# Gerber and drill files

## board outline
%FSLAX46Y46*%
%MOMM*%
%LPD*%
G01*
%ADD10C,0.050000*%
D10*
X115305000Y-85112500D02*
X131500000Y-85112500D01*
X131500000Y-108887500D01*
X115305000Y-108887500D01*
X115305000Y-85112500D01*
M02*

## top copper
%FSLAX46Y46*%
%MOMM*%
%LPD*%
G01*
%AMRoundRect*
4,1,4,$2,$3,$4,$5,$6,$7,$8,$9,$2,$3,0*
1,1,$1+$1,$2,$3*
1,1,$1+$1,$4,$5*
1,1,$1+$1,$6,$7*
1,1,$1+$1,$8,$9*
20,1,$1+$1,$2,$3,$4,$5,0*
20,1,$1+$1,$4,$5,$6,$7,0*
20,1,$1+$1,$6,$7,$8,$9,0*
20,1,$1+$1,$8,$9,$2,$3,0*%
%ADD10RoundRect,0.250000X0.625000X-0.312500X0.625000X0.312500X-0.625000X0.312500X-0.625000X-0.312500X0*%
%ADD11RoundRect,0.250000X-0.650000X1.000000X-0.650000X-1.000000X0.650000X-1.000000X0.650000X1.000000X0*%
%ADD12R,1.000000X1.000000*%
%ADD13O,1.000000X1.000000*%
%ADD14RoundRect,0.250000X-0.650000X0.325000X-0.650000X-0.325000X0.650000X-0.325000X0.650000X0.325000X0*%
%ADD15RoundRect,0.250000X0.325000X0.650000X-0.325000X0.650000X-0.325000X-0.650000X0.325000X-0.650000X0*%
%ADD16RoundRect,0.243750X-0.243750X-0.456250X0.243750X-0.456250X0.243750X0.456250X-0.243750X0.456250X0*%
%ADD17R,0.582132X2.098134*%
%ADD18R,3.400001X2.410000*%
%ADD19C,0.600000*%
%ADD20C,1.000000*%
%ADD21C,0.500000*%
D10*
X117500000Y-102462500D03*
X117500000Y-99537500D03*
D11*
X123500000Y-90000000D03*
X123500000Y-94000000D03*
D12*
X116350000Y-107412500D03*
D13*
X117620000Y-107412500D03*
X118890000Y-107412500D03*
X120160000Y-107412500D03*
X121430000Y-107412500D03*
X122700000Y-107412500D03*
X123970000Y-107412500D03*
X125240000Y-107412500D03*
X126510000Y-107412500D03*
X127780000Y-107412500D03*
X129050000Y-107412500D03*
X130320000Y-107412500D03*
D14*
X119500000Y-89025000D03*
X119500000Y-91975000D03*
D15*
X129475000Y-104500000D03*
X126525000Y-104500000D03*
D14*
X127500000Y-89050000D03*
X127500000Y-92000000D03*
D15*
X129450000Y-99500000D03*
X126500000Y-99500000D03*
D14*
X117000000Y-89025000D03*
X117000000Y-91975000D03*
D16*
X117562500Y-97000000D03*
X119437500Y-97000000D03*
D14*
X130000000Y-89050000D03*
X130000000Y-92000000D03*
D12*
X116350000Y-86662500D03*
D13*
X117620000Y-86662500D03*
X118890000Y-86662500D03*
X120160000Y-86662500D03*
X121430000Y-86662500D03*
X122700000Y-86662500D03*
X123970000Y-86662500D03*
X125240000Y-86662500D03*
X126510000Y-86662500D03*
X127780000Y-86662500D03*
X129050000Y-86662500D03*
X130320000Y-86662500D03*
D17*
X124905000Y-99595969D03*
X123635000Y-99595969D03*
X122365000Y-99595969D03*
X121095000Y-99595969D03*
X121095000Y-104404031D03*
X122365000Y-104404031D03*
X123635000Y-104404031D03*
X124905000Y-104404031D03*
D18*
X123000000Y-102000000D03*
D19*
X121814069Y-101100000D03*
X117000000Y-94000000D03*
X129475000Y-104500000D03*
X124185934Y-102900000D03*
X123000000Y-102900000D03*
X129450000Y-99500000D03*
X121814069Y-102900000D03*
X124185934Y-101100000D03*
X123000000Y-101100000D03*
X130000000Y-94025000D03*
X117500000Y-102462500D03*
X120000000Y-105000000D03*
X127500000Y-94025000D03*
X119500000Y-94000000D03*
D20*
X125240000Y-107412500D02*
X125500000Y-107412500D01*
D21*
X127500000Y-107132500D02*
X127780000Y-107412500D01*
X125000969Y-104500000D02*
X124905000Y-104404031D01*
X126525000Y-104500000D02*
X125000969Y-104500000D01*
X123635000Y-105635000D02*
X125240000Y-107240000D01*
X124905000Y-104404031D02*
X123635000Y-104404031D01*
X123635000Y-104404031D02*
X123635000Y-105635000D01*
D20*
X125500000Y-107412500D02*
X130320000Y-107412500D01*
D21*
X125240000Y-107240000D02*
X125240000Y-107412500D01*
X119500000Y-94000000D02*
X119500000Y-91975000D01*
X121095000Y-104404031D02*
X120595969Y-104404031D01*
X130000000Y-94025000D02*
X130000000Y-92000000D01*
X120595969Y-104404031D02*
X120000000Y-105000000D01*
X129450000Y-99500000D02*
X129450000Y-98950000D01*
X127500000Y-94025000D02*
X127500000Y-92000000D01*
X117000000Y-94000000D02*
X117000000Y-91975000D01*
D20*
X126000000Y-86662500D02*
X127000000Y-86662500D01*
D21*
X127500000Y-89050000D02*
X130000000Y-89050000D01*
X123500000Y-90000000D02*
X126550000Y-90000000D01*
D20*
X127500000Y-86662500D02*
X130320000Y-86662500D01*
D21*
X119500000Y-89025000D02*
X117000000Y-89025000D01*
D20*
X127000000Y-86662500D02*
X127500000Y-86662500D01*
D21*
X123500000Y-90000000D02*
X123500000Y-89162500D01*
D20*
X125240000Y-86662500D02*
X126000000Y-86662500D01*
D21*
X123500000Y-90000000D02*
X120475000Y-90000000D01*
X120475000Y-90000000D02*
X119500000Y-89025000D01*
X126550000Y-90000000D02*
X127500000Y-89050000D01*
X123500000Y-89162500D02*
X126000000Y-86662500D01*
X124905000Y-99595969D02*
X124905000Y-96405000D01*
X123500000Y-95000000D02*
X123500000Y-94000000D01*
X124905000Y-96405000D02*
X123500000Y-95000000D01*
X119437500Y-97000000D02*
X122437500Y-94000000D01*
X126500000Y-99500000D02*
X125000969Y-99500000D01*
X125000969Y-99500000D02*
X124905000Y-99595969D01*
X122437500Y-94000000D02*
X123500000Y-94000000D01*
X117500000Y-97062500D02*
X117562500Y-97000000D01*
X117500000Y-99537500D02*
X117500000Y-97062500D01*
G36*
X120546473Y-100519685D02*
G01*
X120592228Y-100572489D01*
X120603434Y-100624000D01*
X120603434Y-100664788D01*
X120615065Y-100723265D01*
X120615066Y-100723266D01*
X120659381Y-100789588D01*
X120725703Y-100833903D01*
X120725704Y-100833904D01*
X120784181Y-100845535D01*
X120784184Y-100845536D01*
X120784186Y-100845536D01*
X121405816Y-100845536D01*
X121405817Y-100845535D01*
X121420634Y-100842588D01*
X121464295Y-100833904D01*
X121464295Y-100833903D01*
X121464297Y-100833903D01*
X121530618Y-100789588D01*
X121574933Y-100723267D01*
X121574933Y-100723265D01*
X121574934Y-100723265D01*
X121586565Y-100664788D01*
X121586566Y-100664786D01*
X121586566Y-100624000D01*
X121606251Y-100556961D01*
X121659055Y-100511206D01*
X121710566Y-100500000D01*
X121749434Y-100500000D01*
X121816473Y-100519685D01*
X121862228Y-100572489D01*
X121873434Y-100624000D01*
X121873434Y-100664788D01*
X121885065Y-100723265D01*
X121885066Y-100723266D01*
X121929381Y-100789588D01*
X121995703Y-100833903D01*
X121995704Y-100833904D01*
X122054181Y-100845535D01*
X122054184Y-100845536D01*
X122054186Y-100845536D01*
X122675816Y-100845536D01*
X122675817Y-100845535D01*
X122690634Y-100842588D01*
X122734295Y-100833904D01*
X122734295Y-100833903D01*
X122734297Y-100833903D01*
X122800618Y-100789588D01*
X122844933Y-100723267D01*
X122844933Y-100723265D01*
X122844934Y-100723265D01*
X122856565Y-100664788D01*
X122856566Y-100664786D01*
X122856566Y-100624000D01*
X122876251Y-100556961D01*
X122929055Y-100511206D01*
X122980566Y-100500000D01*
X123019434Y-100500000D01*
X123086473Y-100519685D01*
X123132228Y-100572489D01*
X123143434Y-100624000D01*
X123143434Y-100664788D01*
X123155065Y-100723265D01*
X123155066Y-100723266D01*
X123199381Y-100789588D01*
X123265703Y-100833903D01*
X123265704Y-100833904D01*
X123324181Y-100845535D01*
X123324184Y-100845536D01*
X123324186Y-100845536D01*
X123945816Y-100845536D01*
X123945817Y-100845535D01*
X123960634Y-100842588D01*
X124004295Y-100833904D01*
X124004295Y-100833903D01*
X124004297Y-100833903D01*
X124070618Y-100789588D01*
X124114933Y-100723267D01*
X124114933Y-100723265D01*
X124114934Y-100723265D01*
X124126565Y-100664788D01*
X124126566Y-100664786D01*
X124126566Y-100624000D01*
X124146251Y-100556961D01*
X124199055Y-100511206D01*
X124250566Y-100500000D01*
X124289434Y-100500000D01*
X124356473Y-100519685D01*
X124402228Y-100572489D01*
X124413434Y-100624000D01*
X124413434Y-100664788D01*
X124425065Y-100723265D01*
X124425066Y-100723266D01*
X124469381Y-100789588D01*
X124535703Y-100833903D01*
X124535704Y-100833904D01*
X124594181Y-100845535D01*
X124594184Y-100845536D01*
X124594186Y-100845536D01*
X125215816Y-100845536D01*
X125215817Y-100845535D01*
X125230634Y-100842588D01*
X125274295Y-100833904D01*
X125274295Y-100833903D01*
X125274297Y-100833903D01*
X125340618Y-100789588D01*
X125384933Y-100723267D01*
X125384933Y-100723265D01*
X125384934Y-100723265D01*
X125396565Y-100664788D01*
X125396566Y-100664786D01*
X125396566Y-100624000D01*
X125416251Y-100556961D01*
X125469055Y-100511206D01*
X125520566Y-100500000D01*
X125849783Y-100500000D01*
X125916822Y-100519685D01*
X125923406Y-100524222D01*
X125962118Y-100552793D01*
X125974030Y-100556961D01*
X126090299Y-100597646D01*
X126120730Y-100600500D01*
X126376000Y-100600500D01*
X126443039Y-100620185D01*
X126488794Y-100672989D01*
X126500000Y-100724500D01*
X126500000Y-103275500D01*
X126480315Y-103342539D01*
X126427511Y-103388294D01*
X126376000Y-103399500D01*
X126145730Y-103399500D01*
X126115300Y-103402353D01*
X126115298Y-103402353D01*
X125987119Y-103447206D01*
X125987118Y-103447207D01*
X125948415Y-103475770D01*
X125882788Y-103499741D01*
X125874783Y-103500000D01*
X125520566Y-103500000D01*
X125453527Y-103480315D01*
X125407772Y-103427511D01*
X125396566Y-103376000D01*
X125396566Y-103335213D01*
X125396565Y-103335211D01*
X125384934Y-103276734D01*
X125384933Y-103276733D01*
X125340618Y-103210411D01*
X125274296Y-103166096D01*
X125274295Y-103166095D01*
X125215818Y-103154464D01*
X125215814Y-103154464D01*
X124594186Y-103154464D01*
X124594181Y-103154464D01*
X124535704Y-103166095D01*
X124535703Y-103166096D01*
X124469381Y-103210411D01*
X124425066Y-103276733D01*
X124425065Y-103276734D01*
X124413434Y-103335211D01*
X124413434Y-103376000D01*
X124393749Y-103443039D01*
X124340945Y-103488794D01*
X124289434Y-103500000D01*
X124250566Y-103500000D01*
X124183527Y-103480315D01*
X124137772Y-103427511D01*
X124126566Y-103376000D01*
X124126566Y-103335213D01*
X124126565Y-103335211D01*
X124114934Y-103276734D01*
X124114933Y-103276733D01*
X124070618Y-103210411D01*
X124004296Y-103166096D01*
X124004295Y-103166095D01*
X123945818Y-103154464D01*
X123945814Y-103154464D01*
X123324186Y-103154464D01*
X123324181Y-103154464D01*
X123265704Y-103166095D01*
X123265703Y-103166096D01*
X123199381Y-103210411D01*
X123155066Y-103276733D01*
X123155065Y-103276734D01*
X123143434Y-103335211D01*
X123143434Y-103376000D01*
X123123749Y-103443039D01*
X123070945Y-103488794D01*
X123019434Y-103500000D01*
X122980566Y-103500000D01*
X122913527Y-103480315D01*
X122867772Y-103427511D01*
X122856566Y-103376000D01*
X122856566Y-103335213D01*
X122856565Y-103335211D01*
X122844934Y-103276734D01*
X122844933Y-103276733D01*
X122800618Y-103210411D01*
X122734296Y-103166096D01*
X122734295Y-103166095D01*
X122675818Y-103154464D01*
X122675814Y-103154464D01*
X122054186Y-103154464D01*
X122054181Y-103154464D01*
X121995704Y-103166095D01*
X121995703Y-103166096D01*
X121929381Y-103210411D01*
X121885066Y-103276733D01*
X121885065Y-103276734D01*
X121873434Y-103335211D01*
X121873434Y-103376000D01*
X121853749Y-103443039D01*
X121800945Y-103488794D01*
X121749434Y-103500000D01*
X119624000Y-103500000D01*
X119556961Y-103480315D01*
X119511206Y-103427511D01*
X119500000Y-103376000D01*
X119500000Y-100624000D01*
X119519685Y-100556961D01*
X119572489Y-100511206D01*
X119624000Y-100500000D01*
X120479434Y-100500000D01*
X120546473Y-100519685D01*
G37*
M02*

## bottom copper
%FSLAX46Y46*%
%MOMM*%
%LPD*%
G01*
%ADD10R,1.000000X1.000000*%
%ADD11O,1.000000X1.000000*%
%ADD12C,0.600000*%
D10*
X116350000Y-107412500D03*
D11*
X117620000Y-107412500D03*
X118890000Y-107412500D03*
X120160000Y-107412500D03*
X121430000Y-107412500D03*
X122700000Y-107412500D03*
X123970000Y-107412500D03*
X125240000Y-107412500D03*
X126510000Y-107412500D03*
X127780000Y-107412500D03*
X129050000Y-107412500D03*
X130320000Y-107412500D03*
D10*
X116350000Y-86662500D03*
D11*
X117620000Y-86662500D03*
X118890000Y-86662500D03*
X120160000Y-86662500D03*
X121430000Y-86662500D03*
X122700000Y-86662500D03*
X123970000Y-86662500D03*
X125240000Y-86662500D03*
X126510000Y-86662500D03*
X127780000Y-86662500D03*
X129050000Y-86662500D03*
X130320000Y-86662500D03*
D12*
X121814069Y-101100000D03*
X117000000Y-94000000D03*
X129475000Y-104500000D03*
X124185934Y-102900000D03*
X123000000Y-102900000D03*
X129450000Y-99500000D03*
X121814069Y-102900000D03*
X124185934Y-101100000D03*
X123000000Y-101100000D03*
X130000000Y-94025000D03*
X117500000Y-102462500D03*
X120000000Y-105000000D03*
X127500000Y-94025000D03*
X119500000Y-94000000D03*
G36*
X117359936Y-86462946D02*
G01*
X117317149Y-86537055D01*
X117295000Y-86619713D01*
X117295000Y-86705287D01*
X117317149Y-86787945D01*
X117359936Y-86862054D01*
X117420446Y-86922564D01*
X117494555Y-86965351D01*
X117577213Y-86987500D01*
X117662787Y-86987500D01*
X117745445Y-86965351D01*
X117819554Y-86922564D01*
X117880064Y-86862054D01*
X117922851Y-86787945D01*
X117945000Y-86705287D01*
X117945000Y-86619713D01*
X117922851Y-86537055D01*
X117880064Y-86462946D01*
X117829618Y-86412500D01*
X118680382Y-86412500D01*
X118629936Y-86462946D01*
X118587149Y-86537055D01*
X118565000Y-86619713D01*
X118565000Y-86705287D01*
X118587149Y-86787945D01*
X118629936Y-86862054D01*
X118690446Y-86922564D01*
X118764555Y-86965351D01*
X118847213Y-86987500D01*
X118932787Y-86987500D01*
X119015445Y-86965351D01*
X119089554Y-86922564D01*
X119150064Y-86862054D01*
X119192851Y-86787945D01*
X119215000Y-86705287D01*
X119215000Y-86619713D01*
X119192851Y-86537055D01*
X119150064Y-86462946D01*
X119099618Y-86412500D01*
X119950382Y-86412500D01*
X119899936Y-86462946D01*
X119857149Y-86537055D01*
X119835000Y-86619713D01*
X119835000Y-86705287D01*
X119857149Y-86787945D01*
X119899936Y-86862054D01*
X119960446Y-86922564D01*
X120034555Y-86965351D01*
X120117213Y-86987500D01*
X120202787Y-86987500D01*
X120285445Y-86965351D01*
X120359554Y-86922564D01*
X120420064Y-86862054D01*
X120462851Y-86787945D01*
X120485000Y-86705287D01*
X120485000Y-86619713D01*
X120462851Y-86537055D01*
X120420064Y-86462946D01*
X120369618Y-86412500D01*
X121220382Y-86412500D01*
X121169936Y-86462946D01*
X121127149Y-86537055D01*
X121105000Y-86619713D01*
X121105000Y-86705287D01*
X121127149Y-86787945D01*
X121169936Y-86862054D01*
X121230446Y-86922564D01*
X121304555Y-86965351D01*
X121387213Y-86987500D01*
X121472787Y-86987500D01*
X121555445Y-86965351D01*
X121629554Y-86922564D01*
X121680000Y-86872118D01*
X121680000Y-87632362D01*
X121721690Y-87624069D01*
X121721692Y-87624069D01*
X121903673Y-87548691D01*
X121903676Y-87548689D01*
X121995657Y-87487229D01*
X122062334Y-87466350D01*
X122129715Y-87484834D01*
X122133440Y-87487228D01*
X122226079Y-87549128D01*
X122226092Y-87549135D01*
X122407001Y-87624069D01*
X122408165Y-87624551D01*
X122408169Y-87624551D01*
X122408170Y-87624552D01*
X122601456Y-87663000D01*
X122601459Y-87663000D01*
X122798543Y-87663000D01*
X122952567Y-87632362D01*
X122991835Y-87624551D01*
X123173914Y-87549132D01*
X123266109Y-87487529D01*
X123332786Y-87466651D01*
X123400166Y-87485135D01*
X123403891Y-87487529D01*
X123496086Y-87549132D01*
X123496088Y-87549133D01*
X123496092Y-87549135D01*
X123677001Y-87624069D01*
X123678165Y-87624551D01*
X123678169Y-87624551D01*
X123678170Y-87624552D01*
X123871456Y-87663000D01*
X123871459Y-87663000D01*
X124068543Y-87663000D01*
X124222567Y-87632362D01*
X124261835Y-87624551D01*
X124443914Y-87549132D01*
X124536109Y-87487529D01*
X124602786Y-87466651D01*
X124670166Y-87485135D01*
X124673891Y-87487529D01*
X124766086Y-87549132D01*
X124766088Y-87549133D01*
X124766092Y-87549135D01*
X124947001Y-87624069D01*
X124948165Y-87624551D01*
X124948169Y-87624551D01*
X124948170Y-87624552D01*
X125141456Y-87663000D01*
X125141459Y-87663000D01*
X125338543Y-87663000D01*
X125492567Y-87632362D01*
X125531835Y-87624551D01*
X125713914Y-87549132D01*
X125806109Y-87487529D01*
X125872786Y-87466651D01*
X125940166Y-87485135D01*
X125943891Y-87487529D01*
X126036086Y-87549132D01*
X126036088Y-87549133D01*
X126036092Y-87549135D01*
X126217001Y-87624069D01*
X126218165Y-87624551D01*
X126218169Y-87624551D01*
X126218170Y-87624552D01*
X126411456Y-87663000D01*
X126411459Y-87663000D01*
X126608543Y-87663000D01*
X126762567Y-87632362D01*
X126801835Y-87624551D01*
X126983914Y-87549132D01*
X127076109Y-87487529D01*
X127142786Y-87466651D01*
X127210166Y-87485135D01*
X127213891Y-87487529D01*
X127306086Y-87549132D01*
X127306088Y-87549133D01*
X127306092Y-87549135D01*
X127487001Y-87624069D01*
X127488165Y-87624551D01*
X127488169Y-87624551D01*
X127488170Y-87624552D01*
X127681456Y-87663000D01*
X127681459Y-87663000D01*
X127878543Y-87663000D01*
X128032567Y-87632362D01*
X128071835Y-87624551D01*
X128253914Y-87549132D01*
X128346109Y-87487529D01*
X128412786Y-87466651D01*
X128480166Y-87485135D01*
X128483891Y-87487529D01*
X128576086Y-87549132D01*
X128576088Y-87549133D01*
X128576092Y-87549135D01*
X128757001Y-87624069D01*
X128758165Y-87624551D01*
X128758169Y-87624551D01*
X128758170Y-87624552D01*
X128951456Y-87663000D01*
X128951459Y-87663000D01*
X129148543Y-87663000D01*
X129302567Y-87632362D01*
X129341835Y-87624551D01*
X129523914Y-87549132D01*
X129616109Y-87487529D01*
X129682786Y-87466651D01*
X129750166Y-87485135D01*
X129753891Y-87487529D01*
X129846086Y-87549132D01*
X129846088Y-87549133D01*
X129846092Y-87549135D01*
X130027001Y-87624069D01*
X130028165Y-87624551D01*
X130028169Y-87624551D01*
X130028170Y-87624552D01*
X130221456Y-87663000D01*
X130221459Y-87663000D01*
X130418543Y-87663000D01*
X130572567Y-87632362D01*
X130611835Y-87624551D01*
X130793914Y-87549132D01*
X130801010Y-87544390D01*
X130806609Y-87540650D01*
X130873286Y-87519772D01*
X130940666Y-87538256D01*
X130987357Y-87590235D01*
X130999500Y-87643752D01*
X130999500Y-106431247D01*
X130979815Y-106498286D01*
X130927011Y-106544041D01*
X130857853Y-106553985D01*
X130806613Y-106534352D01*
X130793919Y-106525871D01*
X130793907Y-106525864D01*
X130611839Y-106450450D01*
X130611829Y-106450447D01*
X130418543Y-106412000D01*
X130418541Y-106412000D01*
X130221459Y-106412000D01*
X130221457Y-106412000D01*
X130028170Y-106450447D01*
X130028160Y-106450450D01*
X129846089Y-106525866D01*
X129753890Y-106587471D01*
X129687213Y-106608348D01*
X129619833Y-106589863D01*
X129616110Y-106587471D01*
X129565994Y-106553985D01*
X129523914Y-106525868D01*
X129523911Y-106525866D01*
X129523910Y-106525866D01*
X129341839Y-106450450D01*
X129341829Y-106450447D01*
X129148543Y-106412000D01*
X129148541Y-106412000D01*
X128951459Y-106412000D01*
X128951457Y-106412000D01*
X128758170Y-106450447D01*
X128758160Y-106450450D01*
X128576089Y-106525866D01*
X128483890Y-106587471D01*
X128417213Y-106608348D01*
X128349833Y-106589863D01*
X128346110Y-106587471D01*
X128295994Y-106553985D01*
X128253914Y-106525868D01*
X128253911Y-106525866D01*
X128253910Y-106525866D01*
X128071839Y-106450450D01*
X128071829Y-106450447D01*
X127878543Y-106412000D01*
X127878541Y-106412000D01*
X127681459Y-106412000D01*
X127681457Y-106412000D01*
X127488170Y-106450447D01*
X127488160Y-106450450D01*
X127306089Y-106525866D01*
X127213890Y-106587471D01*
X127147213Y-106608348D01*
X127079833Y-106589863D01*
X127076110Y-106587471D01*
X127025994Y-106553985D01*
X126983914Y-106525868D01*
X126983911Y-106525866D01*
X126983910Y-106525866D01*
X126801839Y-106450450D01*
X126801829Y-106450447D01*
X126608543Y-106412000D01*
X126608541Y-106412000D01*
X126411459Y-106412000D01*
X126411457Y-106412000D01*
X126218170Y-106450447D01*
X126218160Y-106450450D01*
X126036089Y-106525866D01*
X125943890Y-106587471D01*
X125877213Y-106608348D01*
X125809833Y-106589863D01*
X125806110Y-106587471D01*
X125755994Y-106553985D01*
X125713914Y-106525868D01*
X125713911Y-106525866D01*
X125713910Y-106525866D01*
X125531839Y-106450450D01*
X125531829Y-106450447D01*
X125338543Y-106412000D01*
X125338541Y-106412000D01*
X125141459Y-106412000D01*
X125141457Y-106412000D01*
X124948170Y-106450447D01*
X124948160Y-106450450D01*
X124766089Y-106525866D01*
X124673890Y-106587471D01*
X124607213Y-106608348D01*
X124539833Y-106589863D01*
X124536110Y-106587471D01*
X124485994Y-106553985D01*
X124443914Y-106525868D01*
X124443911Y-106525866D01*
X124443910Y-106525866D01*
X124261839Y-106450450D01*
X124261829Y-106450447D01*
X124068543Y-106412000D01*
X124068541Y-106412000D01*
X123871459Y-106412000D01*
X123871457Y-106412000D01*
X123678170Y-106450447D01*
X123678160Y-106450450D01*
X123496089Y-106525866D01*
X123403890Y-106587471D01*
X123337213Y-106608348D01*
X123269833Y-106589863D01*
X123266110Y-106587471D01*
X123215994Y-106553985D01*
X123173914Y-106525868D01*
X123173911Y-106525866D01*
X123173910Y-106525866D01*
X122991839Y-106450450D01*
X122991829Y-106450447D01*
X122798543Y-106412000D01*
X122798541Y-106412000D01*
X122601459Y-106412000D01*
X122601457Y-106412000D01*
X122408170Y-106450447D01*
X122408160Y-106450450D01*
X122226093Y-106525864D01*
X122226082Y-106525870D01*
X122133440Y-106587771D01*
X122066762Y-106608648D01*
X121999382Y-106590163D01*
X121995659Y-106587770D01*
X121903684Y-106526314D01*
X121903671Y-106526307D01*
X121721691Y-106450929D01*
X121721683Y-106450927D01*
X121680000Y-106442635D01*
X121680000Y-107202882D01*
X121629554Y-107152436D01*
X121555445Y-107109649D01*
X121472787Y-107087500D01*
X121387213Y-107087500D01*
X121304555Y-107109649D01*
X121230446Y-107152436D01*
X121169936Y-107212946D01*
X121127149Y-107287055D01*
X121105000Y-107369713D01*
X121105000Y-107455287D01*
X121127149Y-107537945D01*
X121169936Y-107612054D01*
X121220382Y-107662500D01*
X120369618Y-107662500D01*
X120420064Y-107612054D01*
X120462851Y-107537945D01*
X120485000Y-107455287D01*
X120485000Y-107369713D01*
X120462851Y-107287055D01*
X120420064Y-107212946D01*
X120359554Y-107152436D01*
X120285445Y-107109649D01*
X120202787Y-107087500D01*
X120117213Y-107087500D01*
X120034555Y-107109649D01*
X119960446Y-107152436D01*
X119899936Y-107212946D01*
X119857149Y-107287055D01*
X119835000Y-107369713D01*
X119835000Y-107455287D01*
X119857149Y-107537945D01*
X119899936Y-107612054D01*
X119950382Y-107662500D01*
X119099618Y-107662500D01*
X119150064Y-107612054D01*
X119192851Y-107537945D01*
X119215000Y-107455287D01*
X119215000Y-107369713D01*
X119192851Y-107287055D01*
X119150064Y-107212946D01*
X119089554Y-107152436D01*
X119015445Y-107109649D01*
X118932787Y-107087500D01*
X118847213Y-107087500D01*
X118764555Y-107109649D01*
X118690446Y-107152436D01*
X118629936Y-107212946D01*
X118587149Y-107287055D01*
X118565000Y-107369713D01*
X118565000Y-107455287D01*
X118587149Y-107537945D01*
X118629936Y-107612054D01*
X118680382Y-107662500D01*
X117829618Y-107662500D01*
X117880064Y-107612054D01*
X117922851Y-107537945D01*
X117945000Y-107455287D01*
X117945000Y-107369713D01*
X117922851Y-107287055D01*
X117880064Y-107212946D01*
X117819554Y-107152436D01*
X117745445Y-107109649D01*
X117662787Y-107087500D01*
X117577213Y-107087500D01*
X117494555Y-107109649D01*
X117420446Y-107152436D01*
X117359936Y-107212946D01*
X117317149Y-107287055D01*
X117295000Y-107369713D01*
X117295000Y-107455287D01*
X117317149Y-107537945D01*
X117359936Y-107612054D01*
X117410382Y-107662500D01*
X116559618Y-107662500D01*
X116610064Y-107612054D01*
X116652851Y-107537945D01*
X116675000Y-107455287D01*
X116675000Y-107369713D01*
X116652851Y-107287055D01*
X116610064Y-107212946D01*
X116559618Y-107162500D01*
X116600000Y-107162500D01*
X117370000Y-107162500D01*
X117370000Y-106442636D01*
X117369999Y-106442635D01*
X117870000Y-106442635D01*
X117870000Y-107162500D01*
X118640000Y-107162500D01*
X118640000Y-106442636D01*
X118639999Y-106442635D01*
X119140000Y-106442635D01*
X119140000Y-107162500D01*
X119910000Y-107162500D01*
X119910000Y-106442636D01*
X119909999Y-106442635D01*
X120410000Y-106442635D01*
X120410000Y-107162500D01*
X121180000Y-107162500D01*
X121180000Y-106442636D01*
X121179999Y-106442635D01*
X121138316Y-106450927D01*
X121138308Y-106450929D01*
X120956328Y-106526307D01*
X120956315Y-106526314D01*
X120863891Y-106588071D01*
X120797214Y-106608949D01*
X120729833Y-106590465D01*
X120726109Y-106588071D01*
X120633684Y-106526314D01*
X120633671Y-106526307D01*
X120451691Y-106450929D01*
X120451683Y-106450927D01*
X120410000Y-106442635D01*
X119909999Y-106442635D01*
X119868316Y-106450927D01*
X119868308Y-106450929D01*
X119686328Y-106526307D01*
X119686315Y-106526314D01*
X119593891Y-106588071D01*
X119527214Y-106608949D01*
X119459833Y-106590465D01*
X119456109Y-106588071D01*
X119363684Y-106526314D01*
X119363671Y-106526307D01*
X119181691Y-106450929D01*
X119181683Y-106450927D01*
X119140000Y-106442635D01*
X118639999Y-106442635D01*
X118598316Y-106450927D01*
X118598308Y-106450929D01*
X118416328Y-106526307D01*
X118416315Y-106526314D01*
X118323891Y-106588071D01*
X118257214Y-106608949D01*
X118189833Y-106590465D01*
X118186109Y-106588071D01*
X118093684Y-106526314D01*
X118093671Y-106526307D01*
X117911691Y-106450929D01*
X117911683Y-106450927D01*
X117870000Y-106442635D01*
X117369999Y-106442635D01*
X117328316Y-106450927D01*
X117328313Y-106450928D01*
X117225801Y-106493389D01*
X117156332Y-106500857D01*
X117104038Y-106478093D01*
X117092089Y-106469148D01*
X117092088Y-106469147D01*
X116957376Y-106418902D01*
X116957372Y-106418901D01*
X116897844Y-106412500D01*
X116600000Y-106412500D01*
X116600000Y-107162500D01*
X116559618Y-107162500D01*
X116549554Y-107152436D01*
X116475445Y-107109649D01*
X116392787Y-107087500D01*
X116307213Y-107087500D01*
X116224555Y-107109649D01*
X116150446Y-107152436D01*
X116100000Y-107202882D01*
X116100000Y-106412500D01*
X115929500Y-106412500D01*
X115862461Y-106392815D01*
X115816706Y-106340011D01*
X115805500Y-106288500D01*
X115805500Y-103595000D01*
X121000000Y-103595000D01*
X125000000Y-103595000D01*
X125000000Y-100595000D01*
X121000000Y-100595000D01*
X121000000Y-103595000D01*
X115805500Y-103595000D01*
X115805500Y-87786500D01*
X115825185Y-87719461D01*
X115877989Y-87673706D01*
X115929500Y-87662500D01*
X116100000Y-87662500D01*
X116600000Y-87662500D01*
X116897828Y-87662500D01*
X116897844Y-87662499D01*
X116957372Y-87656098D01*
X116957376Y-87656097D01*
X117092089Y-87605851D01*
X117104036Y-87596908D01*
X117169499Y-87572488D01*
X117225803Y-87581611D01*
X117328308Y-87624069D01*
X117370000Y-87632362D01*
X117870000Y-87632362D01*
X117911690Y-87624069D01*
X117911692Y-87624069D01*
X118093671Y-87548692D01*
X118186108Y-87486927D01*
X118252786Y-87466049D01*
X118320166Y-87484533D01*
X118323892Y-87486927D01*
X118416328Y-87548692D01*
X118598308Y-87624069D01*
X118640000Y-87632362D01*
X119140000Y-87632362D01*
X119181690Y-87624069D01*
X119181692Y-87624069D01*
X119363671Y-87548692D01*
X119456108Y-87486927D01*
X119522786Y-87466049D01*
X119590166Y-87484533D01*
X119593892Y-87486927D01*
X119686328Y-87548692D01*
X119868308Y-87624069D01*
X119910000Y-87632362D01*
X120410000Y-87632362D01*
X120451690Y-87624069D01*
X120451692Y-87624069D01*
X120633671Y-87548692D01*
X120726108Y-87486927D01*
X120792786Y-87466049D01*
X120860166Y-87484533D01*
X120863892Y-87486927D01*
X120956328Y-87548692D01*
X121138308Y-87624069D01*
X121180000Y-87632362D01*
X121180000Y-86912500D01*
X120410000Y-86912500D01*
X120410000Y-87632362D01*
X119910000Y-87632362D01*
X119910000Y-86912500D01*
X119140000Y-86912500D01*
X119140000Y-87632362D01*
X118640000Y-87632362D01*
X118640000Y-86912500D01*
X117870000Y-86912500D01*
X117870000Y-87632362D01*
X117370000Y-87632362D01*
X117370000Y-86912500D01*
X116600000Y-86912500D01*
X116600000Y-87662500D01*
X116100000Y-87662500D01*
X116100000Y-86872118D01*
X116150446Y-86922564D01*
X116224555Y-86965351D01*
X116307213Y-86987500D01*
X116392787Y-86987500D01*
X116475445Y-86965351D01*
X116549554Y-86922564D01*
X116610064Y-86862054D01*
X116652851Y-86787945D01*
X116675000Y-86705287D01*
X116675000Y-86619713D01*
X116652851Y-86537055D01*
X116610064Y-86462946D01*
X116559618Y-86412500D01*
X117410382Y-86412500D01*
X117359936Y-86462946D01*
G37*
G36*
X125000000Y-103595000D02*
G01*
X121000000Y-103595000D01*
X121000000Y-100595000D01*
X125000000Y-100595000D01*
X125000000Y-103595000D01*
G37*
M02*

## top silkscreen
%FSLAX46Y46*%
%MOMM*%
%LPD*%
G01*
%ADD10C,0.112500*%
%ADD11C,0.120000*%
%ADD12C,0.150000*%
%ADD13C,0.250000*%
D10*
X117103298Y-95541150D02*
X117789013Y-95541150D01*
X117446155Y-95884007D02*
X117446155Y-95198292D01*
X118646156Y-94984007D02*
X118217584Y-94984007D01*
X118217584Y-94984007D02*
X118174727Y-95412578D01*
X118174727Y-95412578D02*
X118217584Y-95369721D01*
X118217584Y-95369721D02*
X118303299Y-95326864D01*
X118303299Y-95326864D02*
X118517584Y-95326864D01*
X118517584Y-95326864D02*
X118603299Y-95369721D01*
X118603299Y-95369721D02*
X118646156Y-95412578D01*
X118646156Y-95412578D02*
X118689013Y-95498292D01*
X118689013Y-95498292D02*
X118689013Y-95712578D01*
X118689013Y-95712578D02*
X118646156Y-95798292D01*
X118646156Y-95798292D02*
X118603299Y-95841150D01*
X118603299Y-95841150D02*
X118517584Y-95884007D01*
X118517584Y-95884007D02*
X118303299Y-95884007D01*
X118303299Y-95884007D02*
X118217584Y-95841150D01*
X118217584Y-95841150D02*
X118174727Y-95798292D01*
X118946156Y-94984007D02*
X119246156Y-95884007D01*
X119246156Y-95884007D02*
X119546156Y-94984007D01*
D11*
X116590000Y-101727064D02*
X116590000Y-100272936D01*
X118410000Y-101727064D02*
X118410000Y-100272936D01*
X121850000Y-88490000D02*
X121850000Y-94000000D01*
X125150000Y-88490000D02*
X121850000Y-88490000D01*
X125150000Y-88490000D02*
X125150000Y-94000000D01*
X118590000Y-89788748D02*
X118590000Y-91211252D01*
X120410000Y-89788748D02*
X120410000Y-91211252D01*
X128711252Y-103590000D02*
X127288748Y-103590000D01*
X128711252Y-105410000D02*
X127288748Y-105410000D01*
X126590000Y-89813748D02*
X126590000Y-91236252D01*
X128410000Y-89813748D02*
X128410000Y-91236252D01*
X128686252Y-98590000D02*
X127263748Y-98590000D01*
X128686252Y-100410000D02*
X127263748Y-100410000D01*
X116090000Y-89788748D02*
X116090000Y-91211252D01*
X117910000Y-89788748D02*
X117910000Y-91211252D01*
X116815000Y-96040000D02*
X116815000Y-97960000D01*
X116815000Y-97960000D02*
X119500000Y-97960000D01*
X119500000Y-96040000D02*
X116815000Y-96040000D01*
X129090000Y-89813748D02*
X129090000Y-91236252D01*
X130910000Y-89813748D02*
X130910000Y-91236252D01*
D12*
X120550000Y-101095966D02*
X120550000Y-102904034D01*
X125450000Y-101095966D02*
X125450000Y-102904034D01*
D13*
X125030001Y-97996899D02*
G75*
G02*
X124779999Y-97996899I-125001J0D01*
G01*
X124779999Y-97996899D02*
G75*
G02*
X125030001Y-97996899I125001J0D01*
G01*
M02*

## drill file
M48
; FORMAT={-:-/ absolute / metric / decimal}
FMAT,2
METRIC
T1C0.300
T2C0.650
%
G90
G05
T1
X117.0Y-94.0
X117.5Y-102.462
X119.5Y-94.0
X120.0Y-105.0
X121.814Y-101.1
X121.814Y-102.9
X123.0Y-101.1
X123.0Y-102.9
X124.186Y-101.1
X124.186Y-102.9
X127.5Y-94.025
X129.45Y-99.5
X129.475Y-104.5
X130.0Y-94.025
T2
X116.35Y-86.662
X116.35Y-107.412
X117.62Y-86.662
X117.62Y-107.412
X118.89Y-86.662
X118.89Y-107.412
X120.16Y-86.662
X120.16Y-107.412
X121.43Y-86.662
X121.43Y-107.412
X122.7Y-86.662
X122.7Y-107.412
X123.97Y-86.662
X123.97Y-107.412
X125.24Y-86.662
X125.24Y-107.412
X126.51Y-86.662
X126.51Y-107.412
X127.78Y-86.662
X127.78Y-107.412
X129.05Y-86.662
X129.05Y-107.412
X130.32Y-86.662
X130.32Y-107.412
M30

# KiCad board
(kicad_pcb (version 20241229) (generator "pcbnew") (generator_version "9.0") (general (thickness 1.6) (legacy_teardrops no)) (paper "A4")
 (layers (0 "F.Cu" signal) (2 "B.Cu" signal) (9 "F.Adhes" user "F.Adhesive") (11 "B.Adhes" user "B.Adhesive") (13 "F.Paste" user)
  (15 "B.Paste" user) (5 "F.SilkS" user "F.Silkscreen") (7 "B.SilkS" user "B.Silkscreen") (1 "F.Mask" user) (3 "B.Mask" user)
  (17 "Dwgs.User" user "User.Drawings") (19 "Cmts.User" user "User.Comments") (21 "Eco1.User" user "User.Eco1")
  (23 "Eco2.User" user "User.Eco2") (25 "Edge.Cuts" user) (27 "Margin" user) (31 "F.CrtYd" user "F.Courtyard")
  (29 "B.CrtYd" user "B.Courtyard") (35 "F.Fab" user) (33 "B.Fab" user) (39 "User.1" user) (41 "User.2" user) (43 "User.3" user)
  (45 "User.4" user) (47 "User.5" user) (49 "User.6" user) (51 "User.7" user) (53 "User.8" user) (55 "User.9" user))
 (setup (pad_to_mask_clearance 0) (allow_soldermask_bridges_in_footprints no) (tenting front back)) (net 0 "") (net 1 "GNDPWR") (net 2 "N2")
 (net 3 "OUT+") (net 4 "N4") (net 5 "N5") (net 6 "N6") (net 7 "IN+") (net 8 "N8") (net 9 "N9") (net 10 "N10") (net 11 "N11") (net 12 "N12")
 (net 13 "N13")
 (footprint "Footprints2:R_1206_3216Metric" (layer "F.Cu") (at 117.5 101 90)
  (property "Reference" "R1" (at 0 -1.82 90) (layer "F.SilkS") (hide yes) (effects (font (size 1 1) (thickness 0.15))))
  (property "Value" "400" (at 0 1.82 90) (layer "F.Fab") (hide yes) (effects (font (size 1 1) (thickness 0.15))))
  (fp_line (start -0.727064 -0.91) (end 0.727064 -0.91) (stroke (width 0.12) (type solid)) (layer "F.SilkS"))
  (fp_line (start -0.727064 0.91) (end 0.727064 0.91) (stroke (width 0.12) (type solid)) (layer "F.SilkS"))
  (pad "1" smd roundrect (at -1.4625 0 90) (size 1.125 1.75) (layers "F.Cu" "F.Mask" "F.Paste") (roundrect_rratio 0.222222) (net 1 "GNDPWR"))
  (pad "2" smd roundrect (at 1.4625 0 90) (size 1.125 1.75) (layers "F.Cu" "F.Mask" "F.Paste") (roundrect_rratio 0.222222) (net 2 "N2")))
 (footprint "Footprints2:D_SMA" (layer "F.Cu") (at 123.5 92 -90)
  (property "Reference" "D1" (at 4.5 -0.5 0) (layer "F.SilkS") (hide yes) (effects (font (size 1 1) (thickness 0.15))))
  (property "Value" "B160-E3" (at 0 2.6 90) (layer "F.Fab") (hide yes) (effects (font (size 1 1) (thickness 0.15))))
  (fp_line (start -3.51 1.65) (end 2 1.65) (stroke (width 0.12) (type solid)) (layer "F.SilkS"))
  (fp_line (start -3.51 -1.65) (end -3.51 1.65) (stroke (width 0.12) (type solid)) (layer "F.SilkS"))
  (fp_line (start -3.51 -1.65) (end 2 -1.65) (stroke (width 0.12) (type solid)) (layer "F.SilkS"))
  (pad "1" smd roundrect (at -2 0 270) (size 2.5 1.8) (layers "F.Cu" "F.Mask" "F.Paste") (roundrect_rratio 0.1388888889) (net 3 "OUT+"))
  (pad "2" smd roundrect (at 2 0 270) (size 2.5 1.8) (layers "F.Cu" "F.Mask" "F.Paste") (roundrect_rratio 0.1388888889) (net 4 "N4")))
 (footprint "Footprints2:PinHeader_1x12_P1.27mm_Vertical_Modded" (layer "F.Cu") (at 115.28 108.9125 90)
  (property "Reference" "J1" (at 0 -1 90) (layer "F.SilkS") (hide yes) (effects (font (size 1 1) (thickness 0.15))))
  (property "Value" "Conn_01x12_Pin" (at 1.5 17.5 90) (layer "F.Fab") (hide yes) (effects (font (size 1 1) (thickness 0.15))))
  (pad "1" thru_hole rect (at 1.5 1.07 90) (size 1 1) (drill 0.65) (layers "*.Cu" "*.Mask") (remove_unused_layers no) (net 1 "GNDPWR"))
  (pad "2" thru_hole oval (at 1.5 2.34 90) (size 1 1) (drill 0.65) (layers "*.Cu" "*.Mask") (remove_unused_layers no) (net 1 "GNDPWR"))
  (pad "3" thru_hole oval (at 1.5 3.61 90) (size 1 1) (drill 0.65) (layers "*.Cu" "*.Mask") (remove_unused_layers no) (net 1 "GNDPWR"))
  (pad "4" thru_hole oval (at 1.5 4.88 90) (size 1 1) (drill 0.65) (layers "*.Cu" "*.Mask") (remove_unused_layers no) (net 1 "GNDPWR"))
  (pad "5" thru_hole oval (at 1.5 6.15 90) (size 1 1) (drill 0.65) (layers "*.Cu" "*.Mask") (remove_unused_layers no) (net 1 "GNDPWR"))
  (pad "6" thru_hole oval (at 1.5 7.42 90) (size 1 1) (drill 0.65) (layers "*.Cu" "*.Mask") (remove_unused_layers no) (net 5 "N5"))
  (pad "7" thru_hole oval (at 1.5 8.69 90) (size 1 1) (drill 0.65) (layers "*.Cu" "*.Mask") (remove_unused_layers no) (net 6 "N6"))
  (pad "8" thru_hole oval (at 1.5 9.96 90) (size 1 1) (drill 0.65) (layers "*.Cu" "*.Mask") (remove_unused_layers no) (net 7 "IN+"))
  (pad "9" thru_hole oval (at 1.5 11.23 90) (size 1 1) (drill 0.65) (layers "*.Cu" "*.Mask") (remove_unused_layers no) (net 7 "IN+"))
  (pad "10" thru_hole oval (at 1.5 12.5 90) (size 1 1) (drill 0.65) (layers "*.Cu" "*.Mask") (remove_unused_layers no) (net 7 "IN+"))
  (pad "11" thru_hole oval (at 1.5 13.77 90) (size 1 1) (drill 0.65) (layers "*.Cu" "*.Mask") (remove_unused_layers no) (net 7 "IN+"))
  (pad "12" thru_hole oval (at 1.5 15.04 90) (size 1 1) (drill 0.65) (layers "*.Cu" "*.Mask") (remove_unused_layers no) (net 7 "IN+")))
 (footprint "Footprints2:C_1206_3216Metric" (layer "F.Cu") (at 119.5 90.5 -90)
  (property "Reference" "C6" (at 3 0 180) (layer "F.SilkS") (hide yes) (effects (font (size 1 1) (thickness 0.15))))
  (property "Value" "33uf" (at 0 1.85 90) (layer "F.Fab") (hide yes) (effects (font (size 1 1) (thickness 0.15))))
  (fp_line (start -0.711252 0.91) (end 0.711252 0.91) (stroke (width 0.12) (type solid)) (layer "F.SilkS"))
  (fp_line (start -0.711252 -0.91) (end 0.711252 -0.91) (stroke (width 0.12) (type solid)) (layer "F.SilkS"))
  (pad "1" smd roundrect (at -1.475 0 270) (size 1.15 1.8) (layers "F.Cu" "F.Mask" "F.Paste") (roundrect_rratio 0.217391) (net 3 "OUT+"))
  (pad "2" smd roundrect (at 1.475 0 270) (size 1.15 1.8) (layers "F.Cu" "F.Mask" "F.Paste") (roundrect_rratio 0.217391) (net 1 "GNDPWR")))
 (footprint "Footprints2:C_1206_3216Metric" (layer "F.Cu") (at 128 104.5 180)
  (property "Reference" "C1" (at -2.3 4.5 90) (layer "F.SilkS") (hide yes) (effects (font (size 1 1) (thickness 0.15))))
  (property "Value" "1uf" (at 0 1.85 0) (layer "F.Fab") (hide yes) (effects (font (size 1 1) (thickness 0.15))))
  (fp_line (start -0.711252 0.91) (end 0.711252 0.91) (stroke (width 0.12) (type solid)) (layer "F.SilkS"))
  (fp_line (start -0.711252 -0.91) (end 0.711252 -0.91) (stroke (width 0.12) (type solid)) (layer "F.SilkS"))
  (pad "1" smd roundrect (at -1.475 0 180) (size 1.15 1.8) (layers "F.Cu" "F.Mask" "F.Paste") (roundrect_rratio 0.217391) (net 1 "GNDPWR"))
  (pad "2" smd roundrect (at 1.475 0 180) (size 1.15 1.8) (layers "F.Cu" "F.Mask" "F.Paste") (roundrect_rratio 0.217391) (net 7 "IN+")))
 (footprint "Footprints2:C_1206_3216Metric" (layer "F.Cu") (at 127.5 90.525 -90)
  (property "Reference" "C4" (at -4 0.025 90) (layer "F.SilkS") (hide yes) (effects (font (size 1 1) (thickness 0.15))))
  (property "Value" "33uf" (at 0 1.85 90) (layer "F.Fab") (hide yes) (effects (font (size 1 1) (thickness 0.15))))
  (fp_line (start -0.711252 0.91) (end 0.711252 0.91) (stroke (width 0.12) (type solid)) (layer "F.SilkS"))
  (fp_line (start -0.711252 -0.91) (end 0.711252 -0.91) (stroke (width 0.12) (type solid)) (layer "F.SilkS"))
  (pad "1" smd roundrect (at -1.475 0 270) (size 1.15 1.8) (layers "F.Cu" "F.Mask" "F.Paste") (roundrect_rratio 0.217391) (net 3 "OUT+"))
  (pad "2" smd roundrect (at 1.475 0 270) (size 1.15 1.8) (layers "F.Cu" "F.Mask" "F.Paste") (roundrect_rratio 0.217391) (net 1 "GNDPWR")))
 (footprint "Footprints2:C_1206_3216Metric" (layer "F.Cu") (at 127.975 99.5 180)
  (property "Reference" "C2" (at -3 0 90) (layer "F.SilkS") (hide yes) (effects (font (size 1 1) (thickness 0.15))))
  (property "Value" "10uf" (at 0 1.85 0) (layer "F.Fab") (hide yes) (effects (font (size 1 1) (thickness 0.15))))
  (fp_line (start -0.711252 0.91) (end 0.711252 0.91) (stroke (width 0.12) (type solid)) (layer "F.SilkS"))
  (fp_line (start -0.711252 -0.91) (end 0.711252 -0.91) (stroke (width 0.12) (type solid)) (layer "F.SilkS"))
  (pad "1" smd roundrect (at -1.475 0 180) (size 1.15 1.8) (layers "F.Cu" "F.Mask" "F.Paste") (roundrect_rratio 0.217391) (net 1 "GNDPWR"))
  (pad "2" smd roundrect (at 1.475 0 180) (size 1.15 1.8) (layers "F.Cu" "F.Mask" "F.Paste") (roundrect_rratio 0.217391) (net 4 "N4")))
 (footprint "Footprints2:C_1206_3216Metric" (layer "F.Cu") (at 117 90.5 -90)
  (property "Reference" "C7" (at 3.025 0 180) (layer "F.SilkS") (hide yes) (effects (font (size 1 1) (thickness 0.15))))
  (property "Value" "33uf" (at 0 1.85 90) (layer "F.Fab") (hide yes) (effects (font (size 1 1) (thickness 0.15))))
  (fp_line (start -0.711252 0.91) (end 0.711252 0.91) (stroke (width 0.12) (type solid)) (layer "F.SilkS"))
  (fp_line (start -0.711252 -0.91) (end 0.711252 -0.91) (stroke (width 0.12) (type solid)) (layer "F.SilkS"))
  (pad "1" smd roundrect (at -1.475 0 270) (size 1.15 1.8) (layers "F.Cu" "F.Mask" "F.Paste") (roundrect_rratio 0.217391) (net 3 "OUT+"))
  (pad "2" smd roundrect (at 1.475 0 270) (size 1.15 1.8) (layers "F.Cu" "F.Mask" "F.Paste") (roundrect_rratio 0.217391) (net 1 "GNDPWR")))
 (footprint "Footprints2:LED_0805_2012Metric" (layer "F.Cu") (at 118.5 97)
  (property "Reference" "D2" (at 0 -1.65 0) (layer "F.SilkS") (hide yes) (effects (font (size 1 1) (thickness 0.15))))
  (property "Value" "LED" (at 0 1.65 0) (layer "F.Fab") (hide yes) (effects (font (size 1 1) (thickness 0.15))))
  (fp_line (start -1.685 -0.96) (end -1.685 0.96) (stroke (width 0.12) (type solid)) (layer "F.SilkS"))
  (fp_line (start -1.685 0.96) (end 1 0.96) (stroke (width 0.12) (type solid)) (layer "F.SilkS"))
  (fp_line (start 1 -0.96) (end -1.685 -0.96) (stroke (width 0.12) (type solid)) (layer "F.SilkS"))
  (pad "1" smd roundrect (at -0.9375 0) (size 0.975 1.4) (layers "F.Cu" "F.Mask" "F.Paste") (roundrect_rratio 0.25) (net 2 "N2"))
  (pad "2" smd roundrect (at 0.9375 0) (size 0.975 1.4) (layers "F.Cu" "F.Mask" "F.Paste") (roundrect_rratio 0.25) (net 4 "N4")))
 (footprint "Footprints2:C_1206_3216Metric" (layer "F.Cu") (at 130 90.525 -90)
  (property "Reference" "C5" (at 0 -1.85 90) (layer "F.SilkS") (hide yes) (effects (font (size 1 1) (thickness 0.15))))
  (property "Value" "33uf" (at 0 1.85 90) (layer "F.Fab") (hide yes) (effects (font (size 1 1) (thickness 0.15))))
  (fp_line (start -0.711252 0.91) (end 0.711252 0.91) (stroke (width 0.12) (type solid)) (layer "F.SilkS"))
  (fp_line (start -0.711252 -0.91) (end 0.711252 -0.91) (stroke (width 0.12) (type solid)) (layer "F.SilkS"))
  (pad "1" smd roundrect (at -1.475 0 270) (size 1.15 1.8) (layers "F.Cu" "F.Mask" "F.Paste") (roundrect_rratio 0.217391) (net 3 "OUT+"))
  (pad "2" smd roundrect (at 1.475 0 270) (size 1.15 1.8) (layers "F.Cu" "F.Mask" "F.Paste") (roundrect_rratio 0.217391) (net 1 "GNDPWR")))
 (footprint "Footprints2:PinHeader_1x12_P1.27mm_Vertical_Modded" (layer "F.Cu") (at 115.28 88.1625 90)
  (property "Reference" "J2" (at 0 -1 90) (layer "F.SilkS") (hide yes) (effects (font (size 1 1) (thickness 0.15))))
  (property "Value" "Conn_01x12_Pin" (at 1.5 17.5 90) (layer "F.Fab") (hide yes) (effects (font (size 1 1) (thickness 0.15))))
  (pad "1" thru_hole rect (at 1.5 1.07 90) (size 1 1) (drill 0.65) (layers "*.Cu" "*.Mask") (remove_unused_layers no) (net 1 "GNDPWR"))
  (pad "2" thru_hole oval (at 1.5 2.34 90) (size 1 1) (drill 0.65) (layers "*.Cu" "*.Mask") (remove_unused_layers no) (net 1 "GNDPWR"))
  (pad "3" thru_hole oval (at 1.5 3.61 90) (size 1 1) (drill 0.65) (layers "*.Cu" "*.Mask") (remove_unused_layers no) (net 1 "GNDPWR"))
  (pad "4" thru_hole oval (at 1.5 4.88 90) (size 1 1) (drill 0.65) (layers "*.Cu" "*.Mask") (remove_unused_layers no) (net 1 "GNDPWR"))
  (pad "5" thru_hole oval (at 1.5 6.15 90) (size 1 1) (drill 0.65) (layers "*.Cu" "*.Mask") (remove_unused_layers no) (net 1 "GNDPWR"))
  (pad "6" thru_hole oval (at 1.5 7.42 90) (size 1 1) (drill 0.65) (layers "*.Cu" "*.Mask") (remove_unused_layers no) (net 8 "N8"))
  (pad "7" thru_hole oval (at 1.5 8.69 90) (size 1 1) (drill 0.65) (layers "*.Cu" "*.Mask") (remove_unused_layers no) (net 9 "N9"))
  (pad "8" thru_hole oval (at 1.5 9.96 90) (size 1 1) (drill 0.65) (layers "*.Cu" "*.Mask") (remove_unused_layers no) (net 3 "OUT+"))
  (pad "9" thru_hole oval (at 1.5 11.23 90) (size 1 1) (drill 0.65) (layers "*.Cu" "*.Mask") (remove_unused_layers no) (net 3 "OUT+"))
  (pad "10" thru_hole oval (at 1.5 12.5 90) (size 1 1) (drill 0.65) (layers "*.Cu" "*.Mask") (remove_unused_layers no) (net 3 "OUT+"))
  (pad "11" thru_hole oval (at 1.5 13.77 90) (size 1 1) (drill 0.65) (layers "*.Cu" "*.Mask") (remove_unused_layers no) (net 3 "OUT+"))
  (pad "12" thru_hole oval (at 1.5 15.04 90) (size 1 1) (drill 0.65) (layers "*.Cu" "*.Mask") (remove_unused_layers no) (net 3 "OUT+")))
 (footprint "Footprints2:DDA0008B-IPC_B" (layer "F.Cu") (at 123 102 -90)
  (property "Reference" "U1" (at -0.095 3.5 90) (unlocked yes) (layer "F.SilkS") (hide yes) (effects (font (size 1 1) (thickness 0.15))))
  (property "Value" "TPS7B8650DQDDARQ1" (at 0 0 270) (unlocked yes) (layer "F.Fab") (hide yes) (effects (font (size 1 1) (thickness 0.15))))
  (fp_line (start -0.904034 2.45) (end 0.904034 2.45) (stroke (width 0.15) (type solid)) (layer "F.SilkS"))
  (fp_line (start -0.904034 -2.45) (end 0.904034 -2.45) (stroke (width 0.15) (type solid)) (layer "F.SilkS"))
  (fp_circle (center -4.003101 -1.905) (end -3.8781 -1.905) (stroke (width 0.25) (type solid)) (fill no) (layer "F.SilkS"))
  (pad "1" smd rect (at -2.404031 -1.905 270) (size 2.098134 0.582132) (layers "F.Cu" "F.Mask" "F.Paste") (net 4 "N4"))
  (pad "2" smd rect (at -2.404031 -0.635 270) (size 2.098134 0.582132) (layers "F.Cu" "F.Mask" "F.Paste") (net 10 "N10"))
  (pad "3" smd rect (at -2.404031 0.635 270) (size 2.098134 0.582132) (layers "F.Cu" "F.Mask" "F.Paste") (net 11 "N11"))
  (pad "4" smd rect (at -2.404031 1.905 270) (size 2.098134 0.582132) (layers "F.Cu" "F.Mask" "F.Paste") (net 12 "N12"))
  (pad "5" smd rect (at 2.404031 1.905 270) (size 2.098134 0.582132) (layers "F.Cu" "F.Mask" "F.Paste") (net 1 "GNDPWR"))
  (pad "6" smd rect (at 2.404031 0.635 270) (size 2.098134 0.582132) (layers "F.Cu" "F.Mask" "F.Paste") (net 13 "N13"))
  (pad "7" smd rect (at 2.404031 -0.635 270) (size 2.098134 0.582132) (layers "F.Cu" "F.Mask" "F.Paste") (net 7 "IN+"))
  (pad "8" smd rect (at 2.404031 -1.905 270) (size 2.098134 0.582132) (layers "F.Cu" "F.Mask" "F.Paste") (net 7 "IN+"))
  (pad "9" smd rect (at 0 0 270) (size 2.41 3.400001) (layers "F.Cu" "F.Mask") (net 1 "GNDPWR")))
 (gr_rect (start 115.305 85.1125) (end 131.5 108.8875) (stroke (width 0.05) (type default)) (fill no) (layer "Edge.Cuts"))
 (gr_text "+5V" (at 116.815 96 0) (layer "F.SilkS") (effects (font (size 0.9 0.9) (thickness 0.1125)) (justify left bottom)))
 (segment (start 125.24 107.4125) (end 125.5 107.4125) (width 1) (layer "F.Cu") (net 7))
 (segment (start 127.5 107.1325) (end 127.78 107.4125) (width 0.5) (layer "F.Cu") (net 7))
 (segment (start 125.000969 104.5) (end 124.905 104.404031) (width 0.5) (layer "F.Cu") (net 7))
 (segment (start 126.525 104.5) (end 125.000969 104.5) (width 0.5) (layer "F.Cu") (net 7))
 (segment (start 123.635 105.635) (end 125.24 107.24) (width 0.5) (layer "F.Cu") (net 7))
 (segment (start 124.905 104.404031) (end 123.635 104.404031) (width 0.5) (layer "F.Cu") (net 7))
 (segment (start 123.635 104.404031) (end 123.635 105.635) (width 0.5) (layer "F.Cu") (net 7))
 (segment (start 125.5 107.4125) (end 130.32 107.4125) (width 1) (layer "F.Cu") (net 7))
 (segment (start 125.24 107.24) (end 125.24 107.4125) (width 0.5) (layer "F.Cu") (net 7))
 (segment (start 119.5 94) (end 119.5 91.975) (width 0.5) (layer "F.Cu") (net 1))
 (segment (start 121.095 104.404031) (end 120.595969 104.404031) (width 0.5) (layer "F.Cu") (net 1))
 (segment (start 130 94.025) (end 130 92) (width 0.5) (layer "F.Cu") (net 1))
 (segment (start 120.595969 104.404031) (end 120 105) (width 0.5) (layer "F.Cu") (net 1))
 (segment (start 129.45 99.5) (end 129.45 98.95) (width 0.5) (layer "F.Cu") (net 1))
 (segment (start 127.5 94.025) (end 127.5 92) (width 0.5) (layer "F.Cu") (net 1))
 (segment (start 117 94) (end 117 91.975) (width 0.5) (layer "F.Cu") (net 1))
 (via (at 121.814069 101.1) (size 0.6) (drill 0.3) (layers "F.Cu" "B.Cu") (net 1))
 (via (at 117 94) (size 0.6) (drill 0.3) (layers "F.Cu" "B.Cu") (free yes) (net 1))
 (via (at 129.475 104.5) (size 0.6) (drill 0.3) (layers "F.Cu" "B.Cu") (free yes) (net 1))
 (via (at 124.185934 102.9) (size 0.6) (drill 0.3) (layers "F.Cu" "B.Cu") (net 1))
 (via (at 123 102.9) (size 0.6) (drill 0.3) (layers "F.Cu" "B.Cu") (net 1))
 (via (at 129.45 99.5) (size 0.6) (drill 0.3) (layers "F.Cu" "B.Cu") (free yes) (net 1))
 (via (at 121.814069 102.9) (size 0.6) (drill 0.3) (layers "F.Cu" "B.Cu") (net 1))
 (via (at 124.185934 101.1) (size 0.6) (drill 0.3) (layers "F.Cu" "B.Cu") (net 1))
 (via (at 123 101.1) (size 0.6) (drill 0.3) (layers "F.Cu" "B.Cu") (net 1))
 (via (at 130 94.025) (size 0.6) (drill 0.3) (layers "F.Cu" "B.Cu") (free yes) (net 1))
 (via (at 117.5 102.4625) (size 0.6) (drill 0.3) (layers "F.Cu" "B.Cu") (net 1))
 (via (at 120 105) (size 0.6) (drill 0.3) (layers "F.Cu" "B.Cu") (free yes) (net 1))
 (via (at 127.5 94.025) (size 0.6) (drill 0.3) (layers "F.Cu" "B.Cu") (free yes) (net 1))
 (via (at 119.5 94) (size 0.6) (drill 0.3) (layers "F.Cu" "B.Cu") (free yes) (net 1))
 (segment (start 126 86.6625) (end 127 86.6625) (width 1) (layer "F.Cu") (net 3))
 (segment (start 127.5 89.05) (end 130 89.05) (width 0.5) (layer "F.Cu") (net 3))
 (segment (start 123.5 90) (end 126.55 90) (width 0.5) (layer "F.Cu") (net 3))
 (segment (start 127.5 86.6625) (end 130.32 86.6625) (width 1) (layer "F.Cu") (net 3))
 (segment (start 119.5 89.025) (end 117 89.025) (width 0.5) (layer "F.Cu") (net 3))
 (segment (start 127 86.6625) (end 127.5 86.6625) (width 1) (layer "F.Cu") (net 3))
 (segment (start 123.5 90) (end 123.5 89.1625) (width 0.5) (layer "F.Cu") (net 3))
 (segment (start 125.24 86.6625) (end 126 86.6625) (width 1) (layer "F.Cu") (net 3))
 (segment (start 123.5 90) (end 120.475 90) (width 0.5) (layer "F.Cu") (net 3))
 (segment (start 120.475 90) (end 119.5 89.025) (width 0.5) (layer "F.Cu") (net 3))
 (segment (start 126.55 90) (end 127.5 89.05) (width 0.5) (layer "F.Cu") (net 3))
 (segment (start 123.5 89.1625) (end 126 86.6625) (width 0.5) (layer "F.Cu") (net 3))
 (segment (start 124.905 99.595969) (end 124.905 96.405) (width 0.5) (layer "F.Cu") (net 4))
 (segment (start 123.5 95) (end 123.5 94) (width 0.5) (layer "F.Cu") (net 4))
 (segment (start 124.905 96.405) (end 123.5 95) (width 0.5) (layer "F.Cu") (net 4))
 (segment (start 119.4375 97) (end 122.4375 94) (width 0.5) (layer "F.Cu") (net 4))
 (segment (start 126.5 99.5) (end 125.000969 99.5) (width 0.5) (layer "F.Cu") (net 4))
 (segment (start 125.000969 99.5) (end 124.905 99.595969) (width 0.5) (layer "F.Cu") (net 4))
 (segment (start 122.4375 94) (end 123.5 94) (width 0.5) (layer "F.Cu") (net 4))
 (segment (start 117.5 97.0625) (end 117.5625 97) (width 0.5) (layer "F.Cu") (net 2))
 (segment (start 117.5 99.5375) (end 117.5 97.0625) (width 0.5) (layer "F.Cu") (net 2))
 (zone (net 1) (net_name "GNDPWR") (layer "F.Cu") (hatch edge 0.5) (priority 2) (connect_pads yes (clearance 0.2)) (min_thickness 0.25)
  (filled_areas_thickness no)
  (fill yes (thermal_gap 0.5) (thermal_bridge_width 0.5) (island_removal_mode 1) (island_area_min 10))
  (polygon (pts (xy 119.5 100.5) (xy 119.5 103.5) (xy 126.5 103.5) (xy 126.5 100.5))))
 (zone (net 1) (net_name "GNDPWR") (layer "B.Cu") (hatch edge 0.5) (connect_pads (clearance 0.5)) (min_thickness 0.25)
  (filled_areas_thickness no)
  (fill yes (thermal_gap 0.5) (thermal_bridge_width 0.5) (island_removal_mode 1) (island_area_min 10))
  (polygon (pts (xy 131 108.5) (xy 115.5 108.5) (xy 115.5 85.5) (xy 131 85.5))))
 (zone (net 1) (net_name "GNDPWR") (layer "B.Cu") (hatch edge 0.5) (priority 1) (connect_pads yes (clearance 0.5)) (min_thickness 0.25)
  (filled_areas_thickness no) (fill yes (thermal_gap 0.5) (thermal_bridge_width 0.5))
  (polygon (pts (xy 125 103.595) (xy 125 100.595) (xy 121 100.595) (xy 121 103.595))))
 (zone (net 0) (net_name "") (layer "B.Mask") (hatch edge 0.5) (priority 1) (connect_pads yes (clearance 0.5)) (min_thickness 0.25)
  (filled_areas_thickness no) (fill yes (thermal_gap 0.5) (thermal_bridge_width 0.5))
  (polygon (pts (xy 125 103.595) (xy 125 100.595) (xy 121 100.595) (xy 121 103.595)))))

